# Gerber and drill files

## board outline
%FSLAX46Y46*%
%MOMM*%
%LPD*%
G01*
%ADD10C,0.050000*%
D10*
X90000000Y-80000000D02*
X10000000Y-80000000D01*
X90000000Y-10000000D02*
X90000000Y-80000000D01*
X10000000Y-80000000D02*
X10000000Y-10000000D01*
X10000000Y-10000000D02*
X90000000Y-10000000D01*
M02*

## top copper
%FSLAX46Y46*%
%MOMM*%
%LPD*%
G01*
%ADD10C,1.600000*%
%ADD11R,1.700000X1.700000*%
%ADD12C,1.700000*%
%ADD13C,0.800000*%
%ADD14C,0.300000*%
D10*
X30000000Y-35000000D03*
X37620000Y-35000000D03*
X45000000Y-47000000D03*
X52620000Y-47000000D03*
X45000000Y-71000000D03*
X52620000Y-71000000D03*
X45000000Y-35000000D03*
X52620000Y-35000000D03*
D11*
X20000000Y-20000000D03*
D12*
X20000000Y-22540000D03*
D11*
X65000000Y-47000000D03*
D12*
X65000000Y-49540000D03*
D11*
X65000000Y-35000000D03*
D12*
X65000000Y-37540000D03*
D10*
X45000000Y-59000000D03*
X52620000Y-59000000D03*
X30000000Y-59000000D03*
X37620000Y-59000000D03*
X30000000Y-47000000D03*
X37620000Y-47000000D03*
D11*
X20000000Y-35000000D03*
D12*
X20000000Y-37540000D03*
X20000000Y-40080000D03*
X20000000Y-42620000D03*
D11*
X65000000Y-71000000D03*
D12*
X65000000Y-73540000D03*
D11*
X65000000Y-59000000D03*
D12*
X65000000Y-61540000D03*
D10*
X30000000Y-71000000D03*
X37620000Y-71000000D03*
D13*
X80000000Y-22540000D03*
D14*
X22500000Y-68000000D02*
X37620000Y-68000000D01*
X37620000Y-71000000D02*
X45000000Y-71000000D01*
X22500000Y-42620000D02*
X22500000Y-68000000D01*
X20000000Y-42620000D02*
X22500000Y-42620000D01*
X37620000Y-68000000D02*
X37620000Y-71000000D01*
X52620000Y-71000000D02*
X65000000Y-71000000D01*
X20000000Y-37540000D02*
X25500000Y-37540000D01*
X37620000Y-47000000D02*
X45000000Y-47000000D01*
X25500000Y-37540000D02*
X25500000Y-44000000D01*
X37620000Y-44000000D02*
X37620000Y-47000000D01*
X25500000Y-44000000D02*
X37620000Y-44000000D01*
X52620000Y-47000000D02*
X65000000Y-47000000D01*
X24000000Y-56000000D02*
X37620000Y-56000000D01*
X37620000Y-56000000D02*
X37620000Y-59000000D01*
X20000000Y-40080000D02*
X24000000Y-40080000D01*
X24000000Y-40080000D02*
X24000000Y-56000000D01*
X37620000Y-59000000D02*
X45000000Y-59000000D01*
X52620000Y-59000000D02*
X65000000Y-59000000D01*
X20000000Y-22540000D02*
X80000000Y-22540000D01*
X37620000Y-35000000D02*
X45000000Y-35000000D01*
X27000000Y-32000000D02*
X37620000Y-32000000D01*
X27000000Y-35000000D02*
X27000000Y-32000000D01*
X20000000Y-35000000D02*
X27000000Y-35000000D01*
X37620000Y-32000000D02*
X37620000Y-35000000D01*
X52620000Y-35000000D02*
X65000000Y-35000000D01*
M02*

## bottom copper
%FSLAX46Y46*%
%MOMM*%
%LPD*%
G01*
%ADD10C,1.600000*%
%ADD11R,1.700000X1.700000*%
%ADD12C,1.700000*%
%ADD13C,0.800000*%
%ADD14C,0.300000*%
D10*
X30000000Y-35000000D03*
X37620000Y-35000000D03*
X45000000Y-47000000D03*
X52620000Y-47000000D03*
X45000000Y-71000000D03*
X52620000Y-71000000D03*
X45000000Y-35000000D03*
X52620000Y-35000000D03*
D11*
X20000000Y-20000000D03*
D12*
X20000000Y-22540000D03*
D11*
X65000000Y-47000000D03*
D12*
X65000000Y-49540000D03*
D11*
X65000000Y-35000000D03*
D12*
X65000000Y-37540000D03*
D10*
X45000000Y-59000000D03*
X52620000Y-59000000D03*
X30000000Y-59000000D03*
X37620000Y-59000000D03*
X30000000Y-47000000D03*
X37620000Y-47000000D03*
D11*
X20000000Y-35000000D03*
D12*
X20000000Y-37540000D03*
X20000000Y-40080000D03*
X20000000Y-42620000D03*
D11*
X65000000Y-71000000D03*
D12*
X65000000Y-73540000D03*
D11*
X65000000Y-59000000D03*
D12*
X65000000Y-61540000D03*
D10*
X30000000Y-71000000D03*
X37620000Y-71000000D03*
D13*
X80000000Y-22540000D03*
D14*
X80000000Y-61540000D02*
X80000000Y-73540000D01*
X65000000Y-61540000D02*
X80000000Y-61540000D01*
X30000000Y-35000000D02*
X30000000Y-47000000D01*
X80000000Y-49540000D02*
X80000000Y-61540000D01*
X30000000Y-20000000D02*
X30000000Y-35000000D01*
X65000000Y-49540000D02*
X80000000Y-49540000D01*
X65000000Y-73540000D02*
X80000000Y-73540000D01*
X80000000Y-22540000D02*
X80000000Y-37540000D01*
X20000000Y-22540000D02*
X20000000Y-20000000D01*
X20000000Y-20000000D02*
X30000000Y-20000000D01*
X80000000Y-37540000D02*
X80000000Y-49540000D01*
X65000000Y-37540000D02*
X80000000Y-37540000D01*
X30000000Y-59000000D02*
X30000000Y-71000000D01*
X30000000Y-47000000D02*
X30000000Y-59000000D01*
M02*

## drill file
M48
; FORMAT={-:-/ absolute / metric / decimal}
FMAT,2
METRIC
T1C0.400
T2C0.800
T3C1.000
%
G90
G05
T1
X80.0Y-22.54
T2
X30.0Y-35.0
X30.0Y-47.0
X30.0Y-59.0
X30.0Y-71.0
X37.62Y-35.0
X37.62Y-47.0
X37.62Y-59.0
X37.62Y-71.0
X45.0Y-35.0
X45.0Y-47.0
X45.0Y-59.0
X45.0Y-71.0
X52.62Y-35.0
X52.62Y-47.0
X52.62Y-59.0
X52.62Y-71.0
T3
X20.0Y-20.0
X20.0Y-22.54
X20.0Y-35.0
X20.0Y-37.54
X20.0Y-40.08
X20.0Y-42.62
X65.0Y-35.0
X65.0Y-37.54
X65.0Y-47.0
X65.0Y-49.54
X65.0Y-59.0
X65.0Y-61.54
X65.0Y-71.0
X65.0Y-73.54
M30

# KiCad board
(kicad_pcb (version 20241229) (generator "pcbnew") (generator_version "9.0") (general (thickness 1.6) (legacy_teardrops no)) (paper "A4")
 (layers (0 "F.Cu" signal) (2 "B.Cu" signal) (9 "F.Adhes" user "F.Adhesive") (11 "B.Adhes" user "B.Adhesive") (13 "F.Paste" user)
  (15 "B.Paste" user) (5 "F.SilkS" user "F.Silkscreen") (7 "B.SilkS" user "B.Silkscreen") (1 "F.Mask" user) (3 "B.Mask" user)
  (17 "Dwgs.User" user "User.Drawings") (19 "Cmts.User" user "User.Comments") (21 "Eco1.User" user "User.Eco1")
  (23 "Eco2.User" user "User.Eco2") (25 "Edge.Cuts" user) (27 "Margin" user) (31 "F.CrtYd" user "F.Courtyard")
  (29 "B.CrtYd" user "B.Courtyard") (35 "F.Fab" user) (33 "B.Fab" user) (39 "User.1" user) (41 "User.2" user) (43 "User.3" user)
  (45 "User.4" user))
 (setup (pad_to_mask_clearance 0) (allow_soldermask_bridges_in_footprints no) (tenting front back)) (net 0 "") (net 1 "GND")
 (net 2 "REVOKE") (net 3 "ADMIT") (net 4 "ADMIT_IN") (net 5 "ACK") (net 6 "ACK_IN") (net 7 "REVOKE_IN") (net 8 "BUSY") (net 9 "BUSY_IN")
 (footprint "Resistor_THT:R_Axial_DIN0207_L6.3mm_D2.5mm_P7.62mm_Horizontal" (layer "F.Cu") (at 30 35)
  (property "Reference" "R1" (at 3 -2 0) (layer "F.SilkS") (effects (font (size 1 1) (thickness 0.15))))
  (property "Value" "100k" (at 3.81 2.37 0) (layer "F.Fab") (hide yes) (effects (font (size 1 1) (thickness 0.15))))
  (pad "1" thru_hole circle (at 0 0) (size 1.6 1.6) (drill 0.8) (layers "*.Cu" "*.Mask") (remove_unused_layers no) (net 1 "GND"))
  (pad "2" thru_hole circle (at 7.62 0) (size 1.6 1.6) (drill 0.8) (layers "*.Cu" "*.Mask") (remove_unused_layers no) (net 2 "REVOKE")))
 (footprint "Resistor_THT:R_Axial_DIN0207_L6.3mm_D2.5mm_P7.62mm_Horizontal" (layer "F.Cu") (at 45 47)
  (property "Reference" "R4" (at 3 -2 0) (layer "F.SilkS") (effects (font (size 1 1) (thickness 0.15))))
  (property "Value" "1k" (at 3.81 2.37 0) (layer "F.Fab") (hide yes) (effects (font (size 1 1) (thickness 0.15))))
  (pad "1" thru_hole circle (at 0 0) (size 1.6 1.6) (drill 0.8) (layers "*.Cu" "*.Mask") (remove_unused_layers no) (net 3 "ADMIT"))
  (pad "2" thru_hole circle (at 7.62 0) (size 1.6 1.6) (drill 0.8) (layers "*.Cu" "*.Mask") (remove_unused_layers no) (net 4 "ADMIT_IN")))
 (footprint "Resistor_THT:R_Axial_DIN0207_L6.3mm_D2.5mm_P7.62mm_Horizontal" (layer "F.Cu") (at 45 71)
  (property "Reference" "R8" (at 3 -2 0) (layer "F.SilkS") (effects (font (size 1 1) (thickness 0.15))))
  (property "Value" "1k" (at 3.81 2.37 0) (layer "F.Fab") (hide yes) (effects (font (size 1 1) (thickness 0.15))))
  (pad "1" thru_hole circle (at 0 0) (size 1.6 1.6) (drill 0.8) (layers "*.Cu" "*.Mask") (remove_unused_layers no) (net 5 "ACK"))
  (pad "2" thru_hole circle (at 7.62 0) (size 1.6 1.6) (drill 0.8) (layers "*.Cu" "*.Mask") (remove_unused_layers no) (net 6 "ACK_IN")))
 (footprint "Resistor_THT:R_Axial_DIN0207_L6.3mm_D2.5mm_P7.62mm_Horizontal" (layer "F.Cu") (at 45 35)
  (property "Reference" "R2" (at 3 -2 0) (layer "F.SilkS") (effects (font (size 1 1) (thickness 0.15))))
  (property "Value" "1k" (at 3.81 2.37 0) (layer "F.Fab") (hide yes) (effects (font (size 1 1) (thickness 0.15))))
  (pad "1" thru_hole circle (at 0 0) (size 1.6 1.6) (drill 0.8) (layers "*.Cu" "*.Mask") (remove_unused_layers no) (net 2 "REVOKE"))
  (pad "2" thru_hole circle (at 7.62 0) (size 1.6 1.6) (drill 0.8) (layers "*.Cu" "*.Mask") (remove_unused_layers no) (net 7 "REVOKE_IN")))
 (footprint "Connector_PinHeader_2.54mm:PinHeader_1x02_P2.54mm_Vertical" (layer "F.Cu") (at 20 20)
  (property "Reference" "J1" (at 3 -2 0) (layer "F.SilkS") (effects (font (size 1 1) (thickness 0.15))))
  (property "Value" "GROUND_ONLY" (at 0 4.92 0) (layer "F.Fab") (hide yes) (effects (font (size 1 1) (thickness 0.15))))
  (pad "1" thru_hole rect (at 0 0) (size 1.7 1.7) (drill 1) (layers "*.Cu" "*.Mask") (remove_unused_layers no) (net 1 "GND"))
  (pad "2" thru_hole circle (at 0 2.54) (size 1.7 1.7) (drill 1) (layers "*.Cu" "*.Mask") (remove_unused_layers no) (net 1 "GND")))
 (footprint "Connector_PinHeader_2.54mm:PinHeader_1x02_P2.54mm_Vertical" (layer "F.Cu") (at 65 47)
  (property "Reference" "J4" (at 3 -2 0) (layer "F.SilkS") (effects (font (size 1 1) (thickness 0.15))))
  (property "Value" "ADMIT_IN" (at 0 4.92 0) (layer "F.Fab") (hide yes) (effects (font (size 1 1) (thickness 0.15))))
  (pad "1" thru_hole rect (at 0 0) (size 1.7 1.7) (drill 1) (layers "*.Cu" "*.Mask") (remove_unused_layers no) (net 4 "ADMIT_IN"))
  (pad "2" thru_hole circle (at 0 2.54) (size 1.7 1.7) (drill 1) (layers "*.Cu" "*.Mask") (remove_unused_layers no) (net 1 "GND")))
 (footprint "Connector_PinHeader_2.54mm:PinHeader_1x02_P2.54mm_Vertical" (layer "F.Cu") (at 65 35)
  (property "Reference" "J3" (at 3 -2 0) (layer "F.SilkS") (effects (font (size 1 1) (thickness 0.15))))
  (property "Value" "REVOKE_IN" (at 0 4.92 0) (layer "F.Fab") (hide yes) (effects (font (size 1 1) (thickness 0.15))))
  (pad "1" thru_hole rect (at 0 0) (size 1.7 1.7) (drill 1) (layers "*.Cu" "*.Mask") (remove_unused_layers no) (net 7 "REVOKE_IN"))
  (pad "2" thru_hole circle (at 0 2.54) (size 1.7 1.7) (drill 1) (layers "*.Cu" "*.Mask") (remove_unused_layers no) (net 1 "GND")))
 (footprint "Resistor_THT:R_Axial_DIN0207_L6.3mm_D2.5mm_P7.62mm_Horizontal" (layer "F.Cu") (at 45 59)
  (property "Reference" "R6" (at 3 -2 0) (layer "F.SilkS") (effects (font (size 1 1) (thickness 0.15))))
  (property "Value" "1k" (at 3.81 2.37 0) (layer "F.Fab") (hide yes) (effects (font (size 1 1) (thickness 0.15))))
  (pad "1" thru_hole circle (at 0 0) (size 1.6 1.6) (drill 0.8) (layers "*.Cu" "*.Mask") (remove_unused_layers no) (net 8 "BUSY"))
  (pad "2" thru_hole circle (at 7.62 0) (size 1.6 1.6) (drill 0.8) (layers "*.Cu" "*.Mask") (remove_unused_layers no) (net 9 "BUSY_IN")))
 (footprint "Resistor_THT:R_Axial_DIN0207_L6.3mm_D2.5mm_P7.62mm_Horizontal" (layer "F.Cu") (at 30 59)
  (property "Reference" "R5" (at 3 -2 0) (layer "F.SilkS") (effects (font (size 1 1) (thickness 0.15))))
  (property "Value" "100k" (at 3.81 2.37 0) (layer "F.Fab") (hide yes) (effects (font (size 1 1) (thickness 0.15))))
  (pad "1" thru_hole circle (at 0 0) (size 1.6 1.6) (drill 0.8) (layers "*.Cu" "*.Mask") (remove_unused_layers no) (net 1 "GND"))
  (pad "2" thru_hole circle (at 7.62 0) (size 1.6 1.6) (drill 0.8) (layers "*.Cu" "*.Mask") (remove_unused_layers no) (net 8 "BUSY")))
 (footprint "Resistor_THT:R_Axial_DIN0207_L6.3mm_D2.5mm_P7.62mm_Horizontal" (layer "F.Cu") (at 30 47)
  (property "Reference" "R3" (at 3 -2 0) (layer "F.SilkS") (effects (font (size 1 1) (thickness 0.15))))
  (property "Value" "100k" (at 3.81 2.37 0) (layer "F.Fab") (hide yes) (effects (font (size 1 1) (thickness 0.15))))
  (pad "1" thru_hole circle (at 0 0) (size 1.6 1.6) (drill 0.8) (layers "*.Cu" "*.Mask") (remove_unused_layers no) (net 1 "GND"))
  (pad "2" thru_hole circle (at 7.62 0) (size 1.6 1.6) (drill 0.8) (layers "*.Cu" "*.Mask") (remove_unused_layers no) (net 3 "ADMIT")))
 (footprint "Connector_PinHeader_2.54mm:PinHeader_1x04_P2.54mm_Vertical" (layer "F.Cu") (at 20 35)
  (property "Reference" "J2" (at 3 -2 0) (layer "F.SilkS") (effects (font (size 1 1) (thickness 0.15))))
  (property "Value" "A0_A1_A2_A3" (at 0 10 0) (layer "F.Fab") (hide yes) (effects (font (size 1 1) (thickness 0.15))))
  (pad "1" thru_hole rect (at 0 0) (size 1.7 1.7) (drill 1) (layers "*.Cu" "*.Mask") (remove_unused_layers no) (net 2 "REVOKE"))
  (pad "2" thru_hole circle (at 0 2.54) (size 1.7 1.7) (drill 1) (layers "*.Cu" "*.Mask") (remove_unused_layers no) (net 3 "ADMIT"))
  (pad "3" thru_hole circle (at 0 5.08) (size 1.7 1.7) (drill 1) (layers "*.Cu" "*.Mask") (remove_unused_layers no) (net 8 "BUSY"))
  (pad "4" thru_hole circle (at 0 7.62) (size 1.7 1.7) (drill 1) (layers "*.Cu" "*.Mask") (remove_unused_layers no) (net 5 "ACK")))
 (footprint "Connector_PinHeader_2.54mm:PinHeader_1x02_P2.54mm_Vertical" (layer "F.Cu") (at 65 71)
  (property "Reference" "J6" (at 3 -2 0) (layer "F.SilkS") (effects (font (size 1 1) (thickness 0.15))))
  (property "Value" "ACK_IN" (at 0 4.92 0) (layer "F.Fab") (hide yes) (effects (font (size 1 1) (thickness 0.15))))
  (pad "1" thru_hole rect (at 0 0) (size 1.7 1.7) (drill 1) (layers "*.Cu" "*.Mask") (remove_unused_layers no) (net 6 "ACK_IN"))
  (pad "2" thru_hole circle (at 0 2.54) (size 1.7 1.7) (drill 1) (layers "*.Cu" "*.Mask") (remove_unused_layers no) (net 1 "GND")))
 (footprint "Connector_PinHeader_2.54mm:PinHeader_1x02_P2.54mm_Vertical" (layer "F.Cu") (at 65 59)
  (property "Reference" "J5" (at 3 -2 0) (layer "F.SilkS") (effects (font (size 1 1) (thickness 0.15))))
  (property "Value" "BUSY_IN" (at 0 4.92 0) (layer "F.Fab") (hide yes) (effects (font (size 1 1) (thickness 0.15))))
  (pad "1" thru_hole rect (at 0 0) (size 1.7 1.7) (drill 1) (layers "*.Cu" "*.Mask") (remove_unused_layers no) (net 9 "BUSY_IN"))
  (pad "2" thru_hole circle (at 0 2.54) (size 1.7 1.7) (drill 1) (layers "*.Cu" "*.Mask") (remove_unused_layers no) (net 1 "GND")))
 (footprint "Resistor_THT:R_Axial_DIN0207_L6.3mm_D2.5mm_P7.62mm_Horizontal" (layer "F.Cu") (at 30 71)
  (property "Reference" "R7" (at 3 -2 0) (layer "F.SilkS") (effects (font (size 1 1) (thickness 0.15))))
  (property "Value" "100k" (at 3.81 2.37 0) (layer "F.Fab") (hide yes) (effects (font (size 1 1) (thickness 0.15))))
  (pad "1" thru_hole circle (at 0 0) (size 1.6 1.6) (drill 0.8) (layers "*.Cu" "*.Mask") (remove_unused_layers no) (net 1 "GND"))
  (pad "2" thru_hole circle (at 7.62 0) (size 1.6 1.6) (drill 0.8) (layers "*.Cu" "*.Mask") (remove_unused_layers no) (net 5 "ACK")))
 (gr_line (start 90 80) (end 10 80) (stroke (width 0.05) (type default)) (layer "Edge.Cuts"))
 (gr_line (start 90 10) (end 90 80) (stroke (width 0.05) (type default)) (layer "Edge.Cuts"))
 (gr_line (start 10 80) (end 10 10) (stroke (width 0.05) (type default)) (layer "Edge.Cuts"))
 (gr_line (start 10 10) (end 90 10) (stroke (width 0.05) (type default)) (layer "Edge.Cuts"))
 (segment (start 22.5 68) (end 37.62 68) (width 0.3) (layer "F.Cu") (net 5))
 (segment (start 37.62 71) (end 45 71) (width 0.3) (layer "F.Cu") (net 5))
 (segment (start 22.5 42.62) (end 22.5 68) (width 0.3) (layer "F.Cu") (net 5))
 (segment (start 20 42.62) (end 22.5 42.62) (width 0.3) (layer "F.Cu") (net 5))
 (segment (start 37.62 68) (end 37.62 71) (width 0.3) (layer "F.Cu") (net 5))
 (segment (start 52.62 71) (end 65 71) (width 0.3) (layer "F.Cu") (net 6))
 (segment (start 20 37.54) (end 25.5 37.54) (width 0.3) (layer "F.Cu") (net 3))
 (segment (start 37.62 47) (end 45 47) (width 0.3) (layer "F.Cu") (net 3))
 (segment (start 25.5 37.54) (end 25.5 44) (width 0.3) (layer "F.Cu") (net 3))
 (segment (start 37.62 44) (end 37.62 47) (width 0.3) (layer "F.Cu") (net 3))
 (segment (start 25.5 44) (end 37.62 44) (width 0.3) (layer "F.Cu") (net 3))
 (segment (start 52.62 47) (end 65 47) (width 0.3) (layer "F.Cu") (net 4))
 (segment (start 24 56) (end 37.62 56) (width 0.3) (layer "F.Cu") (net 8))
 (segment (start 37.62 56) (end 37.62 59) (width 0.3) (layer "F.Cu") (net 8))
 (segment (start 20 40.08) (end 24 40.08) (width 0.3) (layer "F.Cu") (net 8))
 (segment (start 24 40.08) (end 24 56) (width 0.3) (layer "F.Cu") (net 8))
 (segment (start 37.62 59) (end 45 59) (width 0.3) (layer "F.Cu") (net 8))
 (segment (start 52.62 59) (end 65 59) (width 0.3) (layer "F.Cu") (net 9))
 (segment (start 20 22.54) (end 80 22.54) (width 0.3) (layer "F.Cu") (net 1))
 (via (at 80 22.54) (size 0.8) (drill 0.4) (layers "F.Cu" "B.Cu") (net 1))
 (segment (start 80 61.54) (end 80 73.54) (width 0.3) (layer "B.Cu") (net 1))
 (segment (start 65 61.54) (end 80 61.54) (width 0.3) (layer "B.Cu") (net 1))
 (segment (start 30 35) (end 30 47) (width 0.3) (layer "B.Cu") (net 1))
 (segment (start 80 49.54) (end 80 61.54) (width 0.3) (layer "B.Cu") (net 1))
 (segment (start 30 20) (end 30 35) (width 0.3) (layer "B.Cu") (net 1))
 (segment (start 65 49.54) (end 80 49.54) (width 0.3) (layer "B.Cu") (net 1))
 (segment (start 65 73.54) (end 80 73.54) (width 0.3) (layer "B.Cu") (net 1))
 (segment (start 80 22.54) (end 80 37.54) (width 0.3) (layer "B.Cu") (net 1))
 (segment (start 20 22.54) (end 20 20) (width 0.3) (layer "B.Cu") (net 1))
 (segment (start 20 20) (end 30 20) (width 0.3) (layer "B.Cu") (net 1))
 (segment (start 80 37.54) (end 80 49.54) (width 0.3) (layer "B.Cu") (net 1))
 (segment (start 65 37.54) (end 80 37.54) (width 0.3) (layer "B.Cu") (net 1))
 (segment (start 30 59) (end 30 71) (width 0.3) (layer "B.Cu") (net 1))
 (segment (start 30 47) (end 30 59) (width 0.3) (layer "B.Cu") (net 1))
 (segment (start 37.62 35) (end 45 35) (width 0.3) (layer "F.Cu") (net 2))
 (segment (start 27 32) (end 37.62 32) (width 0.3) (layer "F.Cu") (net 2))
 (segment (start 27 35) (end 27 32) (width 0.3) (layer "F.Cu") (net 2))
 (segment (start 20 35) (end 27 35) (width 0.3) (layer "F.Cu") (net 2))
 (segment (start 37.62 32) (end 37.62 35) (width 0.3) (layer "F.Cu") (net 2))
 (segment (start 52.62 35) (end 65 35) (width 0.3) (layer "F.Cu") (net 7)))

